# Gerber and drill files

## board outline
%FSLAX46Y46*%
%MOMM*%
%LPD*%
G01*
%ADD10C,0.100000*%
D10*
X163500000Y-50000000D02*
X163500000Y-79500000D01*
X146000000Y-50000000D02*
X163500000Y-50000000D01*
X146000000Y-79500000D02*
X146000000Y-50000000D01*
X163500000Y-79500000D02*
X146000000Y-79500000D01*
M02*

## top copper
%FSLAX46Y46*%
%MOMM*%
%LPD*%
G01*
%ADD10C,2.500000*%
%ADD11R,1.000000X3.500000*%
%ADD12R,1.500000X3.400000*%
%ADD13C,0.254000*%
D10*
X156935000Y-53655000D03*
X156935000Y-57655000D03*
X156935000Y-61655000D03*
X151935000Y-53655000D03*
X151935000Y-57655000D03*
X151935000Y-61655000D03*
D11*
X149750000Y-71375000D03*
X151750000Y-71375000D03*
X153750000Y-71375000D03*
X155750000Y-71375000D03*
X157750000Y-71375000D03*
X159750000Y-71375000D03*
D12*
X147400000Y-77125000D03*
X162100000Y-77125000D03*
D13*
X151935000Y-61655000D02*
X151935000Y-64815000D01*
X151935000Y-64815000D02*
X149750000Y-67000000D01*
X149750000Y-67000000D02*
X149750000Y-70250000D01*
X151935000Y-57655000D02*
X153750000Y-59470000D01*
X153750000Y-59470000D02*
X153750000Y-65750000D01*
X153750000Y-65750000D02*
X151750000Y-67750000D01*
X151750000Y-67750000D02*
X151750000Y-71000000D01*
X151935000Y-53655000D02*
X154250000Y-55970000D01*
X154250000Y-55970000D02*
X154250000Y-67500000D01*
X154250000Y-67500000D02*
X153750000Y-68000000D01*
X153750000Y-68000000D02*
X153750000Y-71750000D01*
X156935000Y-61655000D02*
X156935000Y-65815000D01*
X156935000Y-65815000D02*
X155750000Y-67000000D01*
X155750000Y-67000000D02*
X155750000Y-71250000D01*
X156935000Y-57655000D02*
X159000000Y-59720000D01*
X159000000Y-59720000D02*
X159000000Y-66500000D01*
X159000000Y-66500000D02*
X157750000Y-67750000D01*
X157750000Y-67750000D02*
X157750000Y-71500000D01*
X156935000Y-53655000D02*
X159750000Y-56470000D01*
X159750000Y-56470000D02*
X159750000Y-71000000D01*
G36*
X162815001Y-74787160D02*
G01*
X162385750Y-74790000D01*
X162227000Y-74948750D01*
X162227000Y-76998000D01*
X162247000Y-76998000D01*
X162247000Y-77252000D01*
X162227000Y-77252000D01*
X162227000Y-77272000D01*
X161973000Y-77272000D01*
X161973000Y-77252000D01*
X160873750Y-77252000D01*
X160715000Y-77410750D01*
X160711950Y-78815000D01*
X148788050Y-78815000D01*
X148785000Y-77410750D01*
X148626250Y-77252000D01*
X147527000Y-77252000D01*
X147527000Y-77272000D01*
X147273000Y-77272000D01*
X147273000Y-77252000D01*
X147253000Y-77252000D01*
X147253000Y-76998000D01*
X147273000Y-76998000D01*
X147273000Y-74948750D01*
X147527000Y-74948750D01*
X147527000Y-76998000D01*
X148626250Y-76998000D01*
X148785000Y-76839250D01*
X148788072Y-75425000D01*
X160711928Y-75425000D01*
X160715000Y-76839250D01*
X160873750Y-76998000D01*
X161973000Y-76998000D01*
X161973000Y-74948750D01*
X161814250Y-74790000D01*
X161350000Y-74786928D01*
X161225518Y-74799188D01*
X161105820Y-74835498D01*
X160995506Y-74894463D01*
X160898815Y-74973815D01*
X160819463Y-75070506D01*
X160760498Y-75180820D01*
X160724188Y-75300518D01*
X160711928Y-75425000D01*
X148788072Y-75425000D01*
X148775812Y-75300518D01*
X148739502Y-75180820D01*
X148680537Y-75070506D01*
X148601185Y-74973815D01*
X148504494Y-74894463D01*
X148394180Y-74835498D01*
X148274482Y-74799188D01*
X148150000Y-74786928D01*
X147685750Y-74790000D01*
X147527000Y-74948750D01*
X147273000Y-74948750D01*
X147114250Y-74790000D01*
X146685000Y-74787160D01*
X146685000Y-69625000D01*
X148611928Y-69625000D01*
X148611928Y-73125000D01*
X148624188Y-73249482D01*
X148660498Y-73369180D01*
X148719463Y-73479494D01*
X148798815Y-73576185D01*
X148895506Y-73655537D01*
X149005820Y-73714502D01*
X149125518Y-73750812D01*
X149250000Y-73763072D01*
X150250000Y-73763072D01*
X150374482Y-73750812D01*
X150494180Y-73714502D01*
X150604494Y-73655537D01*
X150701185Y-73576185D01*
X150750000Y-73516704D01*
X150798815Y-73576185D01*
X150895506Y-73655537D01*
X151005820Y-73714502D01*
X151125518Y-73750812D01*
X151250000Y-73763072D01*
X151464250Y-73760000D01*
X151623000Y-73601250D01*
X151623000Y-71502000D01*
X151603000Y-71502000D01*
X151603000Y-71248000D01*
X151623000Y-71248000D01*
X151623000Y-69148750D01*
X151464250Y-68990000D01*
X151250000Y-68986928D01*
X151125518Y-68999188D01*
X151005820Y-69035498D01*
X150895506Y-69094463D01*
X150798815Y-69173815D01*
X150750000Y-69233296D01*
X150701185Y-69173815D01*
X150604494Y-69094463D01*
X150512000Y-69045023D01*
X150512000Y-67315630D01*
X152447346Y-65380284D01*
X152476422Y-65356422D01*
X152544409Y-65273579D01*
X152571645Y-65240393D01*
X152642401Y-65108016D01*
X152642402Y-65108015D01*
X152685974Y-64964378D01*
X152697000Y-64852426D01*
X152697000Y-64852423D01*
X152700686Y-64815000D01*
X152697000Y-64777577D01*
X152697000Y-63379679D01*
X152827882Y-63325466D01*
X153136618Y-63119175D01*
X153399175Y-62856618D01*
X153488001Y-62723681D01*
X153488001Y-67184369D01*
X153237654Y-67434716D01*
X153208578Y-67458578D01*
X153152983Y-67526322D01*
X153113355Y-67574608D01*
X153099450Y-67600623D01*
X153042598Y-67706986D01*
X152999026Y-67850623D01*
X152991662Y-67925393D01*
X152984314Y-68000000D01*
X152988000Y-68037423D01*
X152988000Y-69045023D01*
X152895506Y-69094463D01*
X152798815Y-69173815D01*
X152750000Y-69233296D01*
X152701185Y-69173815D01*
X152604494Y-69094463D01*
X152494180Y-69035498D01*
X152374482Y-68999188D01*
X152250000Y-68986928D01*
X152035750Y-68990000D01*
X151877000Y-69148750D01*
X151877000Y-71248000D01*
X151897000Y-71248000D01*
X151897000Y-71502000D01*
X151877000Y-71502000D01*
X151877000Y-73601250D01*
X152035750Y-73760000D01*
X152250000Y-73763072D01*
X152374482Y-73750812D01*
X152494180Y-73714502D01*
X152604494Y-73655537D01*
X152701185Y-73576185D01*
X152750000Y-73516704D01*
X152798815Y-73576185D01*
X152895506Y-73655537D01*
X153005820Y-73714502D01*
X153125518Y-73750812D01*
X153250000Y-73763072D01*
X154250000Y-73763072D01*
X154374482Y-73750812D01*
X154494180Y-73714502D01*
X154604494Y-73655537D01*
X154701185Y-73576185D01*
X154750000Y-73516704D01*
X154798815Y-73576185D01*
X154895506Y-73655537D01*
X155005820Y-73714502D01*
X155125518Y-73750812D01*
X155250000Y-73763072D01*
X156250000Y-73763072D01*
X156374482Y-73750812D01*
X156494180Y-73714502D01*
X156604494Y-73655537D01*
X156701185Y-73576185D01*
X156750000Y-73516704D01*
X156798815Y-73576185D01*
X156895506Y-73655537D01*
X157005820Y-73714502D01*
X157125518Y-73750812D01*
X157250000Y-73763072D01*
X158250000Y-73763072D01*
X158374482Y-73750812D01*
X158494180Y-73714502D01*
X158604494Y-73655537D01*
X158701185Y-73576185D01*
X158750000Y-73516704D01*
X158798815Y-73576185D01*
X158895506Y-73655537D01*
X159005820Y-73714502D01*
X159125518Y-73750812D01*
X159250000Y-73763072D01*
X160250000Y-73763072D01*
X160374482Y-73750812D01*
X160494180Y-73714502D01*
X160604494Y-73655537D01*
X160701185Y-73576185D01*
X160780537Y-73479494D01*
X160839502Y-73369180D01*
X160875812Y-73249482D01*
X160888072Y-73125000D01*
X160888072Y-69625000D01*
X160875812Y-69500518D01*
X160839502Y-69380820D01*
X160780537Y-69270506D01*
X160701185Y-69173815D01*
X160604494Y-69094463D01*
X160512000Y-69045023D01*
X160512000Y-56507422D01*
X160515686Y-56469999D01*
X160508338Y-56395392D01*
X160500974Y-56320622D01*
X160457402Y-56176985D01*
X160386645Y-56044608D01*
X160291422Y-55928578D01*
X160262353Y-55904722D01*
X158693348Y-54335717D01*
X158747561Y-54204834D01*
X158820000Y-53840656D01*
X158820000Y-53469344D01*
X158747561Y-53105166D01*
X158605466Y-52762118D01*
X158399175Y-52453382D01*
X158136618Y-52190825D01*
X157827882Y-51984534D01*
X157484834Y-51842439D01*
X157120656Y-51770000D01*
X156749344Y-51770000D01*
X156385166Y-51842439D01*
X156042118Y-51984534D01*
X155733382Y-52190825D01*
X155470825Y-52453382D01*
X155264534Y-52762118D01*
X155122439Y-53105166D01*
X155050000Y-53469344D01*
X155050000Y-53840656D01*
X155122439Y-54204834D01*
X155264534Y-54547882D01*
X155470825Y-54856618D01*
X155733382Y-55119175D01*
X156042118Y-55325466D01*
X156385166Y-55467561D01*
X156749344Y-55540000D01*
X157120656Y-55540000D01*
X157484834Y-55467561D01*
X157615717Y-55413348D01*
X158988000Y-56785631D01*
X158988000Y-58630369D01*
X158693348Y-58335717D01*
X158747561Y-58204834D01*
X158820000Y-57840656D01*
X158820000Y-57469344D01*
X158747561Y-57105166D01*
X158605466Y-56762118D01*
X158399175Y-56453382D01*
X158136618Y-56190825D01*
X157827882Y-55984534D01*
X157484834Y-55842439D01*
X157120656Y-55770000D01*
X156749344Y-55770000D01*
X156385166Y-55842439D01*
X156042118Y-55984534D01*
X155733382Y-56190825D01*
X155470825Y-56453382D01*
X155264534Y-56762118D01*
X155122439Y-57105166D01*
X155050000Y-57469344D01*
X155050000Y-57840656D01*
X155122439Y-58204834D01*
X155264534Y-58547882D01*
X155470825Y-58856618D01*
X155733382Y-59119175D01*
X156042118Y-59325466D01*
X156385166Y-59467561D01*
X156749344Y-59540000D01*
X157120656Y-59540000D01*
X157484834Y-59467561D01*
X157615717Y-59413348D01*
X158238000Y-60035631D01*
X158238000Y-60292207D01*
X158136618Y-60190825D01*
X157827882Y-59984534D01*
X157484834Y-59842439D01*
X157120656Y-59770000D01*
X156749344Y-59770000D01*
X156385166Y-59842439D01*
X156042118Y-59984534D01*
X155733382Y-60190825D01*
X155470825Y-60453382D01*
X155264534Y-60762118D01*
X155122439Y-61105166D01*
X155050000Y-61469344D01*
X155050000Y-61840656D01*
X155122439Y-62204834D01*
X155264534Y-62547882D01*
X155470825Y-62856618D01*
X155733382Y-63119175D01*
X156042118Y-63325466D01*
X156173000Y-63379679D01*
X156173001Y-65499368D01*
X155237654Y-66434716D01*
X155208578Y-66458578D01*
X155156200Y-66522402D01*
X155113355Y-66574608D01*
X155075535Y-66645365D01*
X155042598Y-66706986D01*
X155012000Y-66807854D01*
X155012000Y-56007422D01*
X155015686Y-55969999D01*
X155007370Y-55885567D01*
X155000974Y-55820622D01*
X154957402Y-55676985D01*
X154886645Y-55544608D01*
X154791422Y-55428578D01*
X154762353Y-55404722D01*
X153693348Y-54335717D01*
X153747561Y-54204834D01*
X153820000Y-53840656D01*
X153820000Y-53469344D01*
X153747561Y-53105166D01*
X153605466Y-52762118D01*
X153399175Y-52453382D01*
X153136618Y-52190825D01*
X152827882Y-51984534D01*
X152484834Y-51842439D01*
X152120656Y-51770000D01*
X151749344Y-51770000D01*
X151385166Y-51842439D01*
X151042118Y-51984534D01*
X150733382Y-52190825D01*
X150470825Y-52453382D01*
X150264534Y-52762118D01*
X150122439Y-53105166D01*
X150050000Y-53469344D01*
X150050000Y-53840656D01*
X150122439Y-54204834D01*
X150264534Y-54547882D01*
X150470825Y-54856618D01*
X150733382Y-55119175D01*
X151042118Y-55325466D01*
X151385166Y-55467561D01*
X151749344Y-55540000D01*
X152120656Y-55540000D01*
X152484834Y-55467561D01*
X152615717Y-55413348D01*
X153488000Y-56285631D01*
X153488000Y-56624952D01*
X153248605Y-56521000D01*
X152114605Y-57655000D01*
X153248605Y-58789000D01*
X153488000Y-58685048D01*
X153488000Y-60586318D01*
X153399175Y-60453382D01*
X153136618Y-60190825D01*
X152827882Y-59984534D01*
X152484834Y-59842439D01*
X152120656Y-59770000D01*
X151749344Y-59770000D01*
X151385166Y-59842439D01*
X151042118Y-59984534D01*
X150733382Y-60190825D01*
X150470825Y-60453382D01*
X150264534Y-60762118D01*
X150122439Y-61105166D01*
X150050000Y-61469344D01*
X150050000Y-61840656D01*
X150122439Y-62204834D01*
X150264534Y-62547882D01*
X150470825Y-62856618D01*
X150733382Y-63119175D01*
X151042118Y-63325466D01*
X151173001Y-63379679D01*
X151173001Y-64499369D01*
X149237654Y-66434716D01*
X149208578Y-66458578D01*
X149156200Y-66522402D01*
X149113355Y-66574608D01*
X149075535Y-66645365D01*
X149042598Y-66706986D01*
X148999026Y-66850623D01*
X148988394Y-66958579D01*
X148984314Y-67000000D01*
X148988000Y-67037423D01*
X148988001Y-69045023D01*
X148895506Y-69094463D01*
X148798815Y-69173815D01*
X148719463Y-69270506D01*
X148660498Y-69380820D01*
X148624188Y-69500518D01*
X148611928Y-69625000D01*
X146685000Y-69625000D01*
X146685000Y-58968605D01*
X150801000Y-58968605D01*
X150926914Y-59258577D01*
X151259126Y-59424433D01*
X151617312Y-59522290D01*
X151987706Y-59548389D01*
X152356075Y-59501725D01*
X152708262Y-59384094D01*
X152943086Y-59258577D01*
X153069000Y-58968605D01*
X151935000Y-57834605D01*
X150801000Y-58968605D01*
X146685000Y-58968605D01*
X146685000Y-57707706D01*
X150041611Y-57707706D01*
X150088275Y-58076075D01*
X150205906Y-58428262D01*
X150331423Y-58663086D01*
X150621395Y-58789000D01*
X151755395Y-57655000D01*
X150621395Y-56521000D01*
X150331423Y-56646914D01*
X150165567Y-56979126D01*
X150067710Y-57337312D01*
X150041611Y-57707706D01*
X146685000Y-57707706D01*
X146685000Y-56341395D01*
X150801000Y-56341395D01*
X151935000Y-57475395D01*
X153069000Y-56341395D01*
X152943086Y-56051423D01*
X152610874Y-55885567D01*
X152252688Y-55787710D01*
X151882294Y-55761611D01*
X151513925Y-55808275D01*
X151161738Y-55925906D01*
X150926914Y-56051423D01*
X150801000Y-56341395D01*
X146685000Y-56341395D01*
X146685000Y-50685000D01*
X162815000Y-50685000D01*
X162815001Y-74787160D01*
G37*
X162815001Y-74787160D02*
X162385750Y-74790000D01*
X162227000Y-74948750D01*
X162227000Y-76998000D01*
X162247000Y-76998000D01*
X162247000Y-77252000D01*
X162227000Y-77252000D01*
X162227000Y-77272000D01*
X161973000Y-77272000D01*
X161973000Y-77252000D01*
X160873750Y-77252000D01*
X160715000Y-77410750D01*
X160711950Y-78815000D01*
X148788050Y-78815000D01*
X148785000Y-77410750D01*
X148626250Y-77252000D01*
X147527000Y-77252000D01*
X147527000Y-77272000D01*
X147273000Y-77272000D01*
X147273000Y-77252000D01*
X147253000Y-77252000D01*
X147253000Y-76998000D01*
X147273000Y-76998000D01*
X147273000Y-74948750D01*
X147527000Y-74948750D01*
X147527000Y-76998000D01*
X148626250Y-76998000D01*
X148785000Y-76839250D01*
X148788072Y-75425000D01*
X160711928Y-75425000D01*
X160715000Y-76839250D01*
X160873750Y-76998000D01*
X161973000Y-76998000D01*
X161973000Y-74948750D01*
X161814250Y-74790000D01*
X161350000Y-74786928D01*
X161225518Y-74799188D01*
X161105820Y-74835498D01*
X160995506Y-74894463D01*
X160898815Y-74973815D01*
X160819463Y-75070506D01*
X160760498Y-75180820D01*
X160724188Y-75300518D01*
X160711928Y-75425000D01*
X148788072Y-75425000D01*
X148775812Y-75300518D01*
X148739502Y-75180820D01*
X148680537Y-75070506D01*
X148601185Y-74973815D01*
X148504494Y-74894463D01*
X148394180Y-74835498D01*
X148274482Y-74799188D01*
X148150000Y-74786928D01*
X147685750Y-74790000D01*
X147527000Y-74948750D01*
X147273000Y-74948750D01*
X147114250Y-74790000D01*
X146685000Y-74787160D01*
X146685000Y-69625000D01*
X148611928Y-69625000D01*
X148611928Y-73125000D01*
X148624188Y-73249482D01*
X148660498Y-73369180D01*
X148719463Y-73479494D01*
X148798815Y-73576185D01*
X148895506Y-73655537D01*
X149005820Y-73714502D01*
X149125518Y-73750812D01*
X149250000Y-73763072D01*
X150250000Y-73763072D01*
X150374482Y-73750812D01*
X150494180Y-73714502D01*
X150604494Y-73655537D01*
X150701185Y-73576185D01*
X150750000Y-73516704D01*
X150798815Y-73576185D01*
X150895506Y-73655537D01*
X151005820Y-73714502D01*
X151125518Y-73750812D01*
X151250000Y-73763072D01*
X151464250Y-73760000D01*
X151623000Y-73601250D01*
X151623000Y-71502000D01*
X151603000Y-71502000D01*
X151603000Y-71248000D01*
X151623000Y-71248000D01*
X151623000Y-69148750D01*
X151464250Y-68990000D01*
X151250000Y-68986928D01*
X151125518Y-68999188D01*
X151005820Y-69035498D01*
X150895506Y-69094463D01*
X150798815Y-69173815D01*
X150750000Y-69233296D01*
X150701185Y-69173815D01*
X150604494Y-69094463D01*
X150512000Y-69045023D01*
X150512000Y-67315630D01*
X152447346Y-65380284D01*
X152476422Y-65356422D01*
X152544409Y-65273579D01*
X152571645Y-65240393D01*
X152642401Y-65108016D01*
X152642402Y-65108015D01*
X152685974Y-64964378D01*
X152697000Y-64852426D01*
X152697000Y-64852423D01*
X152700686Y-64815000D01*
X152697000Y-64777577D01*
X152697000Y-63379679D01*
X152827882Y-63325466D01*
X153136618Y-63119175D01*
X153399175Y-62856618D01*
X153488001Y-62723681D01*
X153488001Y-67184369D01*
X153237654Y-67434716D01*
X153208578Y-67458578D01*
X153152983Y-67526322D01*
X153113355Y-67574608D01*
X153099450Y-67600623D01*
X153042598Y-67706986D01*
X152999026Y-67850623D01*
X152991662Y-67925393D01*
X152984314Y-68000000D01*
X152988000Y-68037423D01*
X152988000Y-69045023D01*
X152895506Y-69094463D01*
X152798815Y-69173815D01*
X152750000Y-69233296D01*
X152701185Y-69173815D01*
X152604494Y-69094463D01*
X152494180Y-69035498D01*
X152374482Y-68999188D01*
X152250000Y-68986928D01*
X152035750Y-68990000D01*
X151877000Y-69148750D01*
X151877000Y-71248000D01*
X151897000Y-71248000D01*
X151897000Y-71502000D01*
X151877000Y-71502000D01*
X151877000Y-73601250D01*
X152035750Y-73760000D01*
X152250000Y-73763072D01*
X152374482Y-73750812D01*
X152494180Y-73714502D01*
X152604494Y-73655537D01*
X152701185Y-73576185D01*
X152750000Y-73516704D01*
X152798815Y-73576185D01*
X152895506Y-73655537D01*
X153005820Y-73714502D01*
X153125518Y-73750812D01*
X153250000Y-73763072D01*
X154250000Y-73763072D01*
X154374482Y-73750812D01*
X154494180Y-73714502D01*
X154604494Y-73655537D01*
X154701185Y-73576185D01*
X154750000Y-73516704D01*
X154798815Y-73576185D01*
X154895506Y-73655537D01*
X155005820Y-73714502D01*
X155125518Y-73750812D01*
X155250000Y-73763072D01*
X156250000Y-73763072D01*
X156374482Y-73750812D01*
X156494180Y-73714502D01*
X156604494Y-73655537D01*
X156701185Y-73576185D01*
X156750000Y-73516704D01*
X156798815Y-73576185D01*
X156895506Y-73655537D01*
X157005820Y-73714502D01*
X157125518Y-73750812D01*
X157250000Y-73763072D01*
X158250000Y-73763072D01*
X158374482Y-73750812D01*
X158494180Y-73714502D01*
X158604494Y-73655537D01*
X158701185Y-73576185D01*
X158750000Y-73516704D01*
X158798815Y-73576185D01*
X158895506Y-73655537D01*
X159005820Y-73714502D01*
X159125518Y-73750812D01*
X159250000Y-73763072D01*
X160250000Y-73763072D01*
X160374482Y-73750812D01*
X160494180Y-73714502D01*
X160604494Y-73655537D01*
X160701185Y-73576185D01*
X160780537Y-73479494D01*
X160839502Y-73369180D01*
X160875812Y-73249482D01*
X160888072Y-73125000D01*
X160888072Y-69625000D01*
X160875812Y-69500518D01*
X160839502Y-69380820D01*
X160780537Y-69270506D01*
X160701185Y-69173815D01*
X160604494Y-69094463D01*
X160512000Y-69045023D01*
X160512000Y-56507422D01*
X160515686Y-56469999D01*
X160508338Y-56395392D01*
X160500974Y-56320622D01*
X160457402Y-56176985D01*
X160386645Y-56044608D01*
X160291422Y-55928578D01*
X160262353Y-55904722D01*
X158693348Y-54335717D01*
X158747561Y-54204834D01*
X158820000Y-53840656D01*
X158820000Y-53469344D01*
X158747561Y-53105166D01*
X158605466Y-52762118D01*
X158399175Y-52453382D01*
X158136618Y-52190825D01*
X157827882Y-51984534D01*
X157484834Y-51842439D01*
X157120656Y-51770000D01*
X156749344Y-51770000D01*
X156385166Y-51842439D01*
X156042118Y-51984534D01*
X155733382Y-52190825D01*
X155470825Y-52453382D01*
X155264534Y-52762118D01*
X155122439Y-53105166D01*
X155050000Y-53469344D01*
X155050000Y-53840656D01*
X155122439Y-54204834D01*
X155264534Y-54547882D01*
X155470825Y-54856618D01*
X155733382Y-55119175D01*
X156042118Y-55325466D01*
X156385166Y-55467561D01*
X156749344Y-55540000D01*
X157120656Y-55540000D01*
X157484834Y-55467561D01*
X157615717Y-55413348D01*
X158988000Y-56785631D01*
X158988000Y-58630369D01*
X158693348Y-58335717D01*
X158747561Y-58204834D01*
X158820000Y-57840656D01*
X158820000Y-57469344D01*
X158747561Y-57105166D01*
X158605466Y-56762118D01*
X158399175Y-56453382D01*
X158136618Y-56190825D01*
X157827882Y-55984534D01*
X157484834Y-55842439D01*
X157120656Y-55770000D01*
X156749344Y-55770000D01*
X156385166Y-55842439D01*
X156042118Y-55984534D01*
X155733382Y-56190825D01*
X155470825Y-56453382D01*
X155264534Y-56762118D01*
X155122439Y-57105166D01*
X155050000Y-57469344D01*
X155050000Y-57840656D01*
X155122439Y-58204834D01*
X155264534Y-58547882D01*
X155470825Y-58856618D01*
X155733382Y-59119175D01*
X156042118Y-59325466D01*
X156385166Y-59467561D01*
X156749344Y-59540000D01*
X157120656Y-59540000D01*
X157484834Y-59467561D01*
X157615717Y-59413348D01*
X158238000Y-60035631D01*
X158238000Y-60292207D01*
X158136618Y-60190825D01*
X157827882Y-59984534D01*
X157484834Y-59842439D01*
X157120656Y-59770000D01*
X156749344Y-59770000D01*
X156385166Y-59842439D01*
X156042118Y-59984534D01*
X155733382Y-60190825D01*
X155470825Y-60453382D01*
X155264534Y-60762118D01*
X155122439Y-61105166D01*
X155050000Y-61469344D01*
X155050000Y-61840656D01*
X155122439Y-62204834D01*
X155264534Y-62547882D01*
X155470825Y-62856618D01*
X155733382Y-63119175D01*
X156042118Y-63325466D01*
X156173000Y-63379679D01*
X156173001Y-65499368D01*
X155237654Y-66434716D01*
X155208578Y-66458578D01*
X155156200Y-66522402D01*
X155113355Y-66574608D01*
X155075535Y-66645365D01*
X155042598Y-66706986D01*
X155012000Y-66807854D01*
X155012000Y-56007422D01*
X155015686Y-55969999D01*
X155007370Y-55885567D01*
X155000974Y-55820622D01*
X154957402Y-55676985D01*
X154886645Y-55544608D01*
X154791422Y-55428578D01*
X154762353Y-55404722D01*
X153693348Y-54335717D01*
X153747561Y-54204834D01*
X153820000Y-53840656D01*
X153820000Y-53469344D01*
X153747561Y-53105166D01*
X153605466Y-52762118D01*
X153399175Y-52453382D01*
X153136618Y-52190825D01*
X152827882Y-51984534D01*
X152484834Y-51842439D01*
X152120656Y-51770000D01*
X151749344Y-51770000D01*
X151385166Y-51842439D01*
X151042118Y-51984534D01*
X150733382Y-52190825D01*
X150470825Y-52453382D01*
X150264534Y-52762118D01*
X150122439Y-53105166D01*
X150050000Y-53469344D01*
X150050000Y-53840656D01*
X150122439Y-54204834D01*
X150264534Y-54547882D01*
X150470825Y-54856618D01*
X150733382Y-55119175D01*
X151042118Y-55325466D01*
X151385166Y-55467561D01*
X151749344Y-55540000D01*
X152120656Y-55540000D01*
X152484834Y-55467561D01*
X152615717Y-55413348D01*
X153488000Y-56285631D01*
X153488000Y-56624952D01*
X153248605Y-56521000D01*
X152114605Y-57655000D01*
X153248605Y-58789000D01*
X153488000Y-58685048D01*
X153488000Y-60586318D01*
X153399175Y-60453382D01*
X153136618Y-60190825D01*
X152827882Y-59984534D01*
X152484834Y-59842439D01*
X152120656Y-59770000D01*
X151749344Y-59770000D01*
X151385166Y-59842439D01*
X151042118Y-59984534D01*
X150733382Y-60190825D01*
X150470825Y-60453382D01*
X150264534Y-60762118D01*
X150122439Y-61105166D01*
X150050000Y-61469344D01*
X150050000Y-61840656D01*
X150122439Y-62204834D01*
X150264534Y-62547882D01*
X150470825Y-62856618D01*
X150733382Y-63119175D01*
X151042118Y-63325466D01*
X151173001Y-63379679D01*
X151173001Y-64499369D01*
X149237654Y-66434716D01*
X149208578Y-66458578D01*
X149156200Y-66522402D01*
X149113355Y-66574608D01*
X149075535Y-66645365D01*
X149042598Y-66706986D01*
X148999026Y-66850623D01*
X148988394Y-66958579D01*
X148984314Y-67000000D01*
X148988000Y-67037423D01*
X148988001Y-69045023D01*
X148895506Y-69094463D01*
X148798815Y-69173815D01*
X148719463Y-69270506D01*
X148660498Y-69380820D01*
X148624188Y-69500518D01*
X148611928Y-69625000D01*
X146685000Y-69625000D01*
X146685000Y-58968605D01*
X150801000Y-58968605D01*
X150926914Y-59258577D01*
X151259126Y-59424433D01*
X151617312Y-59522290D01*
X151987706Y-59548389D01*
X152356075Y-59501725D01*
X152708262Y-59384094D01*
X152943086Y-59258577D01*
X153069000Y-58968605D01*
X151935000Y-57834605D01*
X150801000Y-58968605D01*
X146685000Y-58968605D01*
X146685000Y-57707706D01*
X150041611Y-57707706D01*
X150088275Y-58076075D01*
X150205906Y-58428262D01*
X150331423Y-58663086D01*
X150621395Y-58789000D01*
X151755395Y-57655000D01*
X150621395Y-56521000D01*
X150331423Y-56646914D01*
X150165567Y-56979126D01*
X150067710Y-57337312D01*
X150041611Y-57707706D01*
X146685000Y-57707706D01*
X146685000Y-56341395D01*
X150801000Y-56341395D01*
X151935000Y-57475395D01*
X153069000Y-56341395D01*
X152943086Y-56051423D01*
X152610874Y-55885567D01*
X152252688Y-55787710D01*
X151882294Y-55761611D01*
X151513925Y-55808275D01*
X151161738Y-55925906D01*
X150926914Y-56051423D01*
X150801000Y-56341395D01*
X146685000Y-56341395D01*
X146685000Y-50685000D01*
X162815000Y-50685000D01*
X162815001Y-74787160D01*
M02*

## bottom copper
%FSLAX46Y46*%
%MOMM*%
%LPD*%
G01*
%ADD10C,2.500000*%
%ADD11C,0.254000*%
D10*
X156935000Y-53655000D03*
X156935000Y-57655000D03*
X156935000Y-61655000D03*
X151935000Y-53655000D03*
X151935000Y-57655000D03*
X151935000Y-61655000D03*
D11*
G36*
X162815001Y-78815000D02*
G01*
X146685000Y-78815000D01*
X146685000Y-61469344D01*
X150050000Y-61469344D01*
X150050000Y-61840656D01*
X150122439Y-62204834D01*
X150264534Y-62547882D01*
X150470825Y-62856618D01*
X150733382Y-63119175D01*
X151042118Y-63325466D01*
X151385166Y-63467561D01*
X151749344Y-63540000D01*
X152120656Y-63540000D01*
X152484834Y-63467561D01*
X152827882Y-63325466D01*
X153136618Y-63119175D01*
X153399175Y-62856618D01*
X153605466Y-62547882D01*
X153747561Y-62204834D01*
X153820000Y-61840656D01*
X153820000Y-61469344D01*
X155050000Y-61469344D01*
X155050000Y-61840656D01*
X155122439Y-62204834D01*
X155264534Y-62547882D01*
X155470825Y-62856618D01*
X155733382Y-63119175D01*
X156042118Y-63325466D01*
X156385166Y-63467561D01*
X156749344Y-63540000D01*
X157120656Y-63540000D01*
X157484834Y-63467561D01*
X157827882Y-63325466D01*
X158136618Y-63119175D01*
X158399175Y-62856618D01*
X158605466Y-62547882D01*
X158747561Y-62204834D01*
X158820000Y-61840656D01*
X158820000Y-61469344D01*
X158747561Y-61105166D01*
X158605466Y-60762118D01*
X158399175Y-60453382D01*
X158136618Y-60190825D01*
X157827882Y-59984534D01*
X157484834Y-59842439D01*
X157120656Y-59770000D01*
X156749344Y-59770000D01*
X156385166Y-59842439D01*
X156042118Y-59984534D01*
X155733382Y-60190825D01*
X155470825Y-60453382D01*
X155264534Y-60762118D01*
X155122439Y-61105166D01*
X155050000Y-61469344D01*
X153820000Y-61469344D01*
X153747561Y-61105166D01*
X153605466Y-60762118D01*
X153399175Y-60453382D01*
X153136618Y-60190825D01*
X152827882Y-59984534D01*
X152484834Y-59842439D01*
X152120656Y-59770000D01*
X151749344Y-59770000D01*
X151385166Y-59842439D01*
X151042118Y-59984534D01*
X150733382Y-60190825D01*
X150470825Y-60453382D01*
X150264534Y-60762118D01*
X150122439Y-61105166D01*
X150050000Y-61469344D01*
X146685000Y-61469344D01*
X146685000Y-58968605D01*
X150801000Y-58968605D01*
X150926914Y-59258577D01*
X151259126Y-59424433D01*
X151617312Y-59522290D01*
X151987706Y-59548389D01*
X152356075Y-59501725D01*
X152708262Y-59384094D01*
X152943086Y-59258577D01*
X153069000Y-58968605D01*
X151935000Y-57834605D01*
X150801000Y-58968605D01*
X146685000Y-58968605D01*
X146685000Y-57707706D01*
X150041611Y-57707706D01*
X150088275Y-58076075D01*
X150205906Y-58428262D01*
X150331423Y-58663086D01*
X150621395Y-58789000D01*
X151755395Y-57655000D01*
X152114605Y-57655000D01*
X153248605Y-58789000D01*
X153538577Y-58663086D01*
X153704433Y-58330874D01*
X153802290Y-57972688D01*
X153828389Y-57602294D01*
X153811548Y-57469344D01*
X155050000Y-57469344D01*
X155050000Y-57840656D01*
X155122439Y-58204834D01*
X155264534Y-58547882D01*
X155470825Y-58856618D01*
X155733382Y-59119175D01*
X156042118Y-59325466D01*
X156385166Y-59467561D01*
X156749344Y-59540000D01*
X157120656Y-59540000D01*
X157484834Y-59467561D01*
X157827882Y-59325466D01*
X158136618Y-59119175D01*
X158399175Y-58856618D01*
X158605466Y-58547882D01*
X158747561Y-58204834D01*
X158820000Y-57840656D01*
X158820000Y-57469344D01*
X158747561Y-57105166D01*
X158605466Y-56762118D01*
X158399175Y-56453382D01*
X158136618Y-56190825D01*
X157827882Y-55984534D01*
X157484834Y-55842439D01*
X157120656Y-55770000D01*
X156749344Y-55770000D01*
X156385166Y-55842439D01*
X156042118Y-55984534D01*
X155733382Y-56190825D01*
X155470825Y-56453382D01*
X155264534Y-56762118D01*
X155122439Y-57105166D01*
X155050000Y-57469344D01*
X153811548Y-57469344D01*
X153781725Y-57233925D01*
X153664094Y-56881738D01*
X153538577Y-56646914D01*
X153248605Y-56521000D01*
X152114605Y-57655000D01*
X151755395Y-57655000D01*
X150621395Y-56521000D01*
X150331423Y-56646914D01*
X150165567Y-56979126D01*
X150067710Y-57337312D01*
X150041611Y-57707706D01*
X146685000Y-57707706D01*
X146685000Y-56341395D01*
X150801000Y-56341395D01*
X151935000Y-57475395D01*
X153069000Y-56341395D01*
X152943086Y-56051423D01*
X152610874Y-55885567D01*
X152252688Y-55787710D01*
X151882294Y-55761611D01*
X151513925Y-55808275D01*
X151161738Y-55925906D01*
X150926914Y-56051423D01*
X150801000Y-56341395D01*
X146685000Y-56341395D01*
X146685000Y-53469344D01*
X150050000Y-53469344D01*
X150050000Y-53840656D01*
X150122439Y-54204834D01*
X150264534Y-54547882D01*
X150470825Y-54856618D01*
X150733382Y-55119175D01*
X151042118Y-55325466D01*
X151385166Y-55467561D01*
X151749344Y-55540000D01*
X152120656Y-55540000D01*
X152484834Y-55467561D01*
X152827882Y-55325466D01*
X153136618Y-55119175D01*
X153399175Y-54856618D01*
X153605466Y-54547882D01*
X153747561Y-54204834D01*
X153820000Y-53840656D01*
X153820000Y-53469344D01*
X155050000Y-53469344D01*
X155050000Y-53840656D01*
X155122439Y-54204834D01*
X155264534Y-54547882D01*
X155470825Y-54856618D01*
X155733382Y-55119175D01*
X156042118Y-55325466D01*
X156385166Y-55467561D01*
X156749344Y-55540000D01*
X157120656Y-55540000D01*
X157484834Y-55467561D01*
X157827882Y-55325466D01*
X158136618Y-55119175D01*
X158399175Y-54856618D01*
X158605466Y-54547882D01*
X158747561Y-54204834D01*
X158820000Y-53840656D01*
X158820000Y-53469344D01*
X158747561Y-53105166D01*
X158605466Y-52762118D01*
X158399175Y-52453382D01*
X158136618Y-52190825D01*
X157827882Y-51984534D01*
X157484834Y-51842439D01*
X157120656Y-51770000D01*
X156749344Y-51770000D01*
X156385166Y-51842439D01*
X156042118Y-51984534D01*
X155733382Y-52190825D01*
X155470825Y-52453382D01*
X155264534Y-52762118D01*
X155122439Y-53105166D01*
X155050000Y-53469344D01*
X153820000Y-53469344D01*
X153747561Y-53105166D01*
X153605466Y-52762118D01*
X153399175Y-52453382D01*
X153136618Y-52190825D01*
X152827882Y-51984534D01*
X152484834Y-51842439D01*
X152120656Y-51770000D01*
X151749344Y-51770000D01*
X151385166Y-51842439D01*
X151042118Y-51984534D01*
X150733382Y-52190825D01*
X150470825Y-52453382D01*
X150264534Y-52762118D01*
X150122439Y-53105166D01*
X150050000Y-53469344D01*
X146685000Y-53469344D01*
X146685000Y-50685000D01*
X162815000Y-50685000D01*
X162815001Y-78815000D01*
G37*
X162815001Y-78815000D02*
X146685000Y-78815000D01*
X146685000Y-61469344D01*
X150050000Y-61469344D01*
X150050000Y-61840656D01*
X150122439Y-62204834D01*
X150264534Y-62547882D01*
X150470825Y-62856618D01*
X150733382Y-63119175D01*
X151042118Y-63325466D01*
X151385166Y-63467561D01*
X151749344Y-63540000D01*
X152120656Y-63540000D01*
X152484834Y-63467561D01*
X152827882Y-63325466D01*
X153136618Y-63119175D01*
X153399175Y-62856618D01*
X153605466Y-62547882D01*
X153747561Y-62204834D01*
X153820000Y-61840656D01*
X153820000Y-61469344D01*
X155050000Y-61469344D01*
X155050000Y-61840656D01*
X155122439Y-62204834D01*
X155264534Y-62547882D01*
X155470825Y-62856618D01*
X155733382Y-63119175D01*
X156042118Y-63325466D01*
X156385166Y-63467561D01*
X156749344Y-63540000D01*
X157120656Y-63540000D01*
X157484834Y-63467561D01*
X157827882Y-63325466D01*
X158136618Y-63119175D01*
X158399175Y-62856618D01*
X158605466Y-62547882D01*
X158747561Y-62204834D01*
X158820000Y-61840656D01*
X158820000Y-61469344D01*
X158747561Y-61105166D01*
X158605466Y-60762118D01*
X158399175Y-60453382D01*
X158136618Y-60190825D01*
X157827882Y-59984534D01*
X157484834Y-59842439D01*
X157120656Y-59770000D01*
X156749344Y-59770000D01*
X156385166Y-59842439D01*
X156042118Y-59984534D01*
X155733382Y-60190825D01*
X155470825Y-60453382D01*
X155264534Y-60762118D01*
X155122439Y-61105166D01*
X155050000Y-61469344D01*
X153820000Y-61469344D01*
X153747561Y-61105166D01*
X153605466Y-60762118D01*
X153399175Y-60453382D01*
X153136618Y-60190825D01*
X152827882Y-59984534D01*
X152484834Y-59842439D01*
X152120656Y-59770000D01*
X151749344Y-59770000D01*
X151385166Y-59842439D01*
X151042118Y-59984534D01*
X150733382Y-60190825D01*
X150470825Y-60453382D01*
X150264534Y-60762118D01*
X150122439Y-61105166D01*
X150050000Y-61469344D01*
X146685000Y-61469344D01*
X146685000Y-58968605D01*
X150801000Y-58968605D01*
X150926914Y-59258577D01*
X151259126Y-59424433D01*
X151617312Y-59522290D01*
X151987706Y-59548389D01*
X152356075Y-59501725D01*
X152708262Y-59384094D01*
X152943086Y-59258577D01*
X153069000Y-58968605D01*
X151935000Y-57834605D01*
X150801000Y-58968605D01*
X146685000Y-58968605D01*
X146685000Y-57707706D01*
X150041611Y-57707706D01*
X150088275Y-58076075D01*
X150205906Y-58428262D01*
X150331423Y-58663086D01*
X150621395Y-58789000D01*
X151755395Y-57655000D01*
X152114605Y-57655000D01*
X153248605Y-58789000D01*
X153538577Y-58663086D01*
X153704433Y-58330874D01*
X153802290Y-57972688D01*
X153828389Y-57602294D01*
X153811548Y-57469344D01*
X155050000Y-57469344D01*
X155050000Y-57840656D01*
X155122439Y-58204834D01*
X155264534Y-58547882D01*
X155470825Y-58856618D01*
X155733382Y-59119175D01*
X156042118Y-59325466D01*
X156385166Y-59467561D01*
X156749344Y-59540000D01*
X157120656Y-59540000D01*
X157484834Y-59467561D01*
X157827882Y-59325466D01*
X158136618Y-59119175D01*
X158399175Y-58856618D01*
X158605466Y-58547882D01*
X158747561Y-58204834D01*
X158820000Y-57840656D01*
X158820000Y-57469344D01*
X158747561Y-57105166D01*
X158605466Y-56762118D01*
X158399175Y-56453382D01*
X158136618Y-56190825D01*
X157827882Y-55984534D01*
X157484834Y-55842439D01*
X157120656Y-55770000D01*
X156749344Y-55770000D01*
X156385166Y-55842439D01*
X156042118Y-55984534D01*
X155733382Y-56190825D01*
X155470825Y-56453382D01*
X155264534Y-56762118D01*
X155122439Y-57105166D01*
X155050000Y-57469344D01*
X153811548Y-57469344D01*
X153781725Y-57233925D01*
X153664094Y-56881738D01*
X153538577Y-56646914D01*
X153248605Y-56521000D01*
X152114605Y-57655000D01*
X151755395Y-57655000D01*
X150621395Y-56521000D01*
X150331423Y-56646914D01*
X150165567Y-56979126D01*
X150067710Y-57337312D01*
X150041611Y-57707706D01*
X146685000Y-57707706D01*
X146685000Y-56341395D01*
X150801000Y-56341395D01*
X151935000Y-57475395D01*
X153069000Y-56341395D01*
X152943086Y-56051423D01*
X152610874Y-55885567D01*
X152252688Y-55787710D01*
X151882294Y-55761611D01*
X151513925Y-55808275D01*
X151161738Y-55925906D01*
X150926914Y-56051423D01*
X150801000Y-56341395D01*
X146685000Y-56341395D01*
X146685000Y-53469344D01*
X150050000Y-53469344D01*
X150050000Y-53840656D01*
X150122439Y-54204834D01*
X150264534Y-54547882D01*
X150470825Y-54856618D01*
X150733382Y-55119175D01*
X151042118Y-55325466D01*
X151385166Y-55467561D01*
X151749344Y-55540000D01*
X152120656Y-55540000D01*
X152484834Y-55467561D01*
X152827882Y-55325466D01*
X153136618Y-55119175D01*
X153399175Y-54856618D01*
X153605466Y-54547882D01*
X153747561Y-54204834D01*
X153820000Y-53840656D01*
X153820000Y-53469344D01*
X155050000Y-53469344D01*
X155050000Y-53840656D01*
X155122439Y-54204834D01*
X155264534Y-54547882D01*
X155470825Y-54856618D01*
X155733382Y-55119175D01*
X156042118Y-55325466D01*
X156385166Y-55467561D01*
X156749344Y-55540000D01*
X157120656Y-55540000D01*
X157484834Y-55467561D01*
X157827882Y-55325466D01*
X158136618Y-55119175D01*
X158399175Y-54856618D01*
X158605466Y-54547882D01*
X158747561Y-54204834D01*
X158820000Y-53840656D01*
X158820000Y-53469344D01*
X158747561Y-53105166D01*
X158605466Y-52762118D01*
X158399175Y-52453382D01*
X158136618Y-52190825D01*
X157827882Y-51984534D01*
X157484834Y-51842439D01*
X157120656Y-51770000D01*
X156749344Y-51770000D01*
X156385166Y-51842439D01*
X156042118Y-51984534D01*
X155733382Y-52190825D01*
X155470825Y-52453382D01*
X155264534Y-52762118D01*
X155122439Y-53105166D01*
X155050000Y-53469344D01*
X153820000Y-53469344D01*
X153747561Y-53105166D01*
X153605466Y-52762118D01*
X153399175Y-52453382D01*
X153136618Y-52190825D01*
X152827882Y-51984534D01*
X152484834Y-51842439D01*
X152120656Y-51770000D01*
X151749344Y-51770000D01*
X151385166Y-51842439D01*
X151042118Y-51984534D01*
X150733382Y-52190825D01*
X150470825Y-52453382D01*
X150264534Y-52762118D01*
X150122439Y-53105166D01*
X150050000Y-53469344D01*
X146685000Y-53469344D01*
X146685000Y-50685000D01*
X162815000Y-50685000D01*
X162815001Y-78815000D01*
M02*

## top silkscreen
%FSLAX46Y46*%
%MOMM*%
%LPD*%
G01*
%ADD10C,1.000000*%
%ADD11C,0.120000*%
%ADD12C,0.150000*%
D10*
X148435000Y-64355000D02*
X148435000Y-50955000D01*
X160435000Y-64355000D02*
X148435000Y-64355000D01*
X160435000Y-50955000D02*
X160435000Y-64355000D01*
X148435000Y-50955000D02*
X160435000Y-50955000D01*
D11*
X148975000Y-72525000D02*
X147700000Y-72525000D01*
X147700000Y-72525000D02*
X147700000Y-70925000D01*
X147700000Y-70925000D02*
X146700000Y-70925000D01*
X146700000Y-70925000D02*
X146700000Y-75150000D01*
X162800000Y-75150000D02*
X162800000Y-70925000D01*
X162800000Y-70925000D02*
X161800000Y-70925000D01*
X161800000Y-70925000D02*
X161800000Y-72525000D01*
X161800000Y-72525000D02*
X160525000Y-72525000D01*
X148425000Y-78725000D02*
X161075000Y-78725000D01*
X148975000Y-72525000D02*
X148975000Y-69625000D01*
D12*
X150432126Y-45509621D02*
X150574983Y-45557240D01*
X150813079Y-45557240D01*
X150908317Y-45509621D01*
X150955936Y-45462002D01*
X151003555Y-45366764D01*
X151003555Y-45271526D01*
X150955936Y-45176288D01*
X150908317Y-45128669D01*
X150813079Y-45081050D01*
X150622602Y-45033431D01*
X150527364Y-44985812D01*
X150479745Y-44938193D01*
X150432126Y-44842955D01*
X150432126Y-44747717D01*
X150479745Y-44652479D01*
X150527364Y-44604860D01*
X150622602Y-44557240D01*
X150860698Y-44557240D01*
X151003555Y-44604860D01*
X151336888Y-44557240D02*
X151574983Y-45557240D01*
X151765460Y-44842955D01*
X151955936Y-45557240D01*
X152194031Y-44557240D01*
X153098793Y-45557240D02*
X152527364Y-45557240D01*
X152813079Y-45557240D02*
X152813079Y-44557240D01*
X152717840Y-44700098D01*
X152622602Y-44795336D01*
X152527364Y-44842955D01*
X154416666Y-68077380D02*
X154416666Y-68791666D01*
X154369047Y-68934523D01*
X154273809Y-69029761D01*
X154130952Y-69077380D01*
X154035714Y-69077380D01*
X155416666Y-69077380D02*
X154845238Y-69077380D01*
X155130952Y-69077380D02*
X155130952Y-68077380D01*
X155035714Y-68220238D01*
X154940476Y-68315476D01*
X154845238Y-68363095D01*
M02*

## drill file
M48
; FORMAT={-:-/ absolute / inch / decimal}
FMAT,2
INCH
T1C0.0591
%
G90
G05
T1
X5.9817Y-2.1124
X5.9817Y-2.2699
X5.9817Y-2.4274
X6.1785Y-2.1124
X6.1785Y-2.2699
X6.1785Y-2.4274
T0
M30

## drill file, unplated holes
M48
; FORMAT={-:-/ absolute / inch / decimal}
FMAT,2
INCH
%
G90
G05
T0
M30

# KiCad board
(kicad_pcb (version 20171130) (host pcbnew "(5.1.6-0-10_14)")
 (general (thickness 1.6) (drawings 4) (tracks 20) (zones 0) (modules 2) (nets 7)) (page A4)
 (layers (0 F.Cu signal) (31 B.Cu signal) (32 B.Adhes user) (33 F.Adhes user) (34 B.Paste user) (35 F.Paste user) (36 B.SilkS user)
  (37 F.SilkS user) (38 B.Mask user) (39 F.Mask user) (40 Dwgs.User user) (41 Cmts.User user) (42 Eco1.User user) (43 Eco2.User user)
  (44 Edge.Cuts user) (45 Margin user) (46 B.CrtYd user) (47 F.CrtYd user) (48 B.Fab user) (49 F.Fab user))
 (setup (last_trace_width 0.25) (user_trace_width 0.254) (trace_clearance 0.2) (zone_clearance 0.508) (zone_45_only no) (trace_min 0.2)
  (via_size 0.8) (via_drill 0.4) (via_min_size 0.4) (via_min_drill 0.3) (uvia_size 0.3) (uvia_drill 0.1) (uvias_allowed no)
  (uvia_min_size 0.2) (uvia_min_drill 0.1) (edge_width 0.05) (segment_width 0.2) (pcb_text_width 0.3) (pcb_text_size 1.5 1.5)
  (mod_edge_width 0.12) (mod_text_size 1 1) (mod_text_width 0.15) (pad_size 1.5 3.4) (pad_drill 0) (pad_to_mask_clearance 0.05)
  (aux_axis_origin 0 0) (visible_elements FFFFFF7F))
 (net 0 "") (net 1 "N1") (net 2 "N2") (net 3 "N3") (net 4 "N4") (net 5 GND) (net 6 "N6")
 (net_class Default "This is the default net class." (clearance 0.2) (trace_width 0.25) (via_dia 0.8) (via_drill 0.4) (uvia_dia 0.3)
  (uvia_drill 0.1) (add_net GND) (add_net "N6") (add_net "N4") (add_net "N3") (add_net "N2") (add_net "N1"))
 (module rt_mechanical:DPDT (layer F.Cu) (at 154.435 57.655)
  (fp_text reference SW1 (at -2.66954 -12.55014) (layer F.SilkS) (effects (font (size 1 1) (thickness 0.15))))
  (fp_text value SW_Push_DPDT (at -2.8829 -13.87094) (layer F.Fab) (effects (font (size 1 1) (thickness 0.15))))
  (fp_line (start -6 6.7) (end -6 -6.7) (layer F.SilkS) (width 1))
  (fp_line (start 6 6.7) (end -6 6.7) (layer F.SilkS) (width 1))
  (fp_line (start 6 -6.7) (end 6 6.7) (layer F.SilkS) (width 1))
  (fp_line (start -6 -6.7) (end 6 -6.7) (layer F.SilkS) (width 1))
  (pad 6 thru_hole circle (at 2.5 -4) (size 2.5 2.5) (drill 1.5) (layers *.Cu *.Mask) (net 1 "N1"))
  (pad 5 thru_hole circle (at 2.5 0) (size 2.5 2.5) (drill 1.5) (layers *.Cu *.Mask) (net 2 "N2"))
  (pad 4 thru_hole circle (at 2.5 4) (size 2.5 2.5) (drill 1.5) (layers *.Cu *.Mask) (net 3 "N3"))
  (pad 3 thru_hole circle (at -2.5 -4) (size 2.5 2.5) (drill 1.5) (layers *.Cu *.Mask) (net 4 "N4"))
  (pad 2 thru_hole circle (at -2.5 0) (size 2.5 2.5) (drill 1.5) (layers *.Cu *.Mask) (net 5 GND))
  (pad 1 thru_hole circle (at -2.5 4) (size 2.5 2.5) (drill 1.5) (layers *.Cu *.Mask) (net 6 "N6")))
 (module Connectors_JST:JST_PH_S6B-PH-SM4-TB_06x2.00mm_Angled (layer F.Cu) (at 154.75 74.25)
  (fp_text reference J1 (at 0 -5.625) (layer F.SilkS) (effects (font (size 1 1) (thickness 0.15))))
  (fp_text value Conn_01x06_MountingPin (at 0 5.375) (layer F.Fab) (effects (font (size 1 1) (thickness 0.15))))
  (fp_line (start -5.775 -1.725) (end -7.05 -1.725) (layer F.SilkS) (width 0.12))
  (fp_line (start -7.05 -1.725) (end -7.05 -3.325) (layer F.SilkS) (width 0.12))
  (fp_line (start -7.05 -3.325) (end -8.05 -3.325) (layer F.SilkS) (width 0.12))
  (fp_line (start -8.05 -3.325) (end -8.05 0.9) (layer F.SilkS) (width 0.12))
  (fp_line (start 8.05 0.9) (end 8.05 -3.325) (layer F.SilkS) (width 0.12))
  (fp_line (start 8.05 -3.325) (end 7.05 -3.325) (layer F.SilkS) (width 0.12))
  (fp_line (start 7.05 -3.325) (end 7.05 -1.725) (layer F.SilkS) (width 0.12))
  (fp_line (start 7.05 -1.725) (end 5.775 -1.725) (layer F.SilkS) (width 0.12))
  (fp_line (start -6.325 4.475) (end 6.325 4.475) (layer F.SilkS) (width 0.12))
  (fp_line (start -5.775 -1.725) (end -5.775 -4.625) (layer F.SilkS) (width 0.12))
  (pad 1 smd rect (at -5 -2.875) (size 1 3.5) (layers F.Cu F.Paste F.Mask) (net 6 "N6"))
  (pad 2 smd rect (at -3 -2.875) (size 1 3.5) (layers F.Cu F.Paste F.Mask) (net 5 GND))
  (pad 3 smd rect (at -1 -2.875) (size 1 3.5) (layers F.Cu F.Paste F.Mask) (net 4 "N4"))
  (pad 4 smd rect (at 1 -2.875) (size 1 3.5) (layers F.Cu F.Paste F.Mask) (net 3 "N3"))
  (pad 5 smd rect (at 3 -2.875) (size 1 3.5) (layers F.Cu F.Paste F.Mask) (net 2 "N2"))
  (pad 6 smd rect (at 5 -2.875) (size 1 3.5) (layers F.Cu F.Paste F.Mask) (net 1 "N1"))
  (pad "" smd rect (at -7.35 2.875) (size 1.5 3.4) (layers F.Cu F.Paste F.Mask) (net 5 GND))
  (pad "" smd rect (at 7.35 2.875) (size 1.5 3.4) (layers F.Cu F.Paste F.Mask) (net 5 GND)))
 (gr_line (start 163.5 50) (end 163.5 79.5) (layer Edge.Cuts) (width 0.1))
 (gr_line (start 146 50) (end 163.5 50) (layer Edge.Cuts) (width 0.1))
 (gr_line (start 146 79.5) (end 146 50) (layer Edge.Cuts) (width 0.1))
 (gr_line (start 163.5 79.5) (end 146 79.5) (layer Edge.Cuts) (width 0.1))
 (segment (start 151.935 61.655) (end 151.935 64.815) (width 0.254) (layer F.Cu) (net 6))
 (segment (start 151.935 64.815) (end 149.75 67) (width 0.254) (layer F.Cu) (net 6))
 (segment (start 149.75 67) (end 149.75 70.25) (width 0.254) (layer F.Cu) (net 6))
 (segment (start 151.935 57.655) (end 153.75 59.47) (width 0.254) (layer F.Cu) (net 5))
 (segment (start 153.75 59.47) (end 153.75 65.75) (width 0.254) (layer F.Cu) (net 5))
 (segment (start 153.75 65.75) (end 151.75 67.75) (width 0.254) (layer F.Cu) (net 5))
 (segment (start 151.75 67.75) (end 151.75 71) (width 0.254) (layer F.Cu) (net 5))
 (segment (start 151.935 53.655) (end 154.25 55.97) (width 0.254) (layer F.Cu) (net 4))
 (segment (start 154.25 55.97) (end 154.25 67.5) (width 0.254) (layer F.Cu) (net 4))
 (segment (start 154.25 67.5) (end 153.75 68) (width 0.254) (layer F.Cu) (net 4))
 (segment (start 153.75 68) (end 153.75 71.75) (width 0.254) (layer F.Cu) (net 4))
 (segment (start 156.935 61.655) (end 156.935 65.815) (width 0.254) (layer F.Cu) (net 3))
 (segment (start 156.935 65.815) (end 155.75 67) (width 0.254) (layer F.Cu) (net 3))
 (segment (start 155.75 67) (end 155.75 71.25) (width 0.254) (layer F.Cu) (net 3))
 (segment (start 156.935 57.655) (end 159 59.72) (width 0.254) (layer F.Cu) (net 2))
 (segment (start 159 59.72) (end 159 66.5) (width 0.254) (layer F.Cu) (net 2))
 (segment (start 159 66.5) (end 157.75 67.75) (width 0.254) (layer F.Cu) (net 2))
 (segment (start 157.75 67.75) (end 157.75 71.5) (width 0.254) (layer F.Cu) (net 2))
 (segment (start 156.935 53.655) (end 159.75 56.47) (width 0.254) (layer F.Cu) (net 1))
 (segment (start 159.75 56.47) (end 159.75 71) (width 0.254) (layer F.Cu) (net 1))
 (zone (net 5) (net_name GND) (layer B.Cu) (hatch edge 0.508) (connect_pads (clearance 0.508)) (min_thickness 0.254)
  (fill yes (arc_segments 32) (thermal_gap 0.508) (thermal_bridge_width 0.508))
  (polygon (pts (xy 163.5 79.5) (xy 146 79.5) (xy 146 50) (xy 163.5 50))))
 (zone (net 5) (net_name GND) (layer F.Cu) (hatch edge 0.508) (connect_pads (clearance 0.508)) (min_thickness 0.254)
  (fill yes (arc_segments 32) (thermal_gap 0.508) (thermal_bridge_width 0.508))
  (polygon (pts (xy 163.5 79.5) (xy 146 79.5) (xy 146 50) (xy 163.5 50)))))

